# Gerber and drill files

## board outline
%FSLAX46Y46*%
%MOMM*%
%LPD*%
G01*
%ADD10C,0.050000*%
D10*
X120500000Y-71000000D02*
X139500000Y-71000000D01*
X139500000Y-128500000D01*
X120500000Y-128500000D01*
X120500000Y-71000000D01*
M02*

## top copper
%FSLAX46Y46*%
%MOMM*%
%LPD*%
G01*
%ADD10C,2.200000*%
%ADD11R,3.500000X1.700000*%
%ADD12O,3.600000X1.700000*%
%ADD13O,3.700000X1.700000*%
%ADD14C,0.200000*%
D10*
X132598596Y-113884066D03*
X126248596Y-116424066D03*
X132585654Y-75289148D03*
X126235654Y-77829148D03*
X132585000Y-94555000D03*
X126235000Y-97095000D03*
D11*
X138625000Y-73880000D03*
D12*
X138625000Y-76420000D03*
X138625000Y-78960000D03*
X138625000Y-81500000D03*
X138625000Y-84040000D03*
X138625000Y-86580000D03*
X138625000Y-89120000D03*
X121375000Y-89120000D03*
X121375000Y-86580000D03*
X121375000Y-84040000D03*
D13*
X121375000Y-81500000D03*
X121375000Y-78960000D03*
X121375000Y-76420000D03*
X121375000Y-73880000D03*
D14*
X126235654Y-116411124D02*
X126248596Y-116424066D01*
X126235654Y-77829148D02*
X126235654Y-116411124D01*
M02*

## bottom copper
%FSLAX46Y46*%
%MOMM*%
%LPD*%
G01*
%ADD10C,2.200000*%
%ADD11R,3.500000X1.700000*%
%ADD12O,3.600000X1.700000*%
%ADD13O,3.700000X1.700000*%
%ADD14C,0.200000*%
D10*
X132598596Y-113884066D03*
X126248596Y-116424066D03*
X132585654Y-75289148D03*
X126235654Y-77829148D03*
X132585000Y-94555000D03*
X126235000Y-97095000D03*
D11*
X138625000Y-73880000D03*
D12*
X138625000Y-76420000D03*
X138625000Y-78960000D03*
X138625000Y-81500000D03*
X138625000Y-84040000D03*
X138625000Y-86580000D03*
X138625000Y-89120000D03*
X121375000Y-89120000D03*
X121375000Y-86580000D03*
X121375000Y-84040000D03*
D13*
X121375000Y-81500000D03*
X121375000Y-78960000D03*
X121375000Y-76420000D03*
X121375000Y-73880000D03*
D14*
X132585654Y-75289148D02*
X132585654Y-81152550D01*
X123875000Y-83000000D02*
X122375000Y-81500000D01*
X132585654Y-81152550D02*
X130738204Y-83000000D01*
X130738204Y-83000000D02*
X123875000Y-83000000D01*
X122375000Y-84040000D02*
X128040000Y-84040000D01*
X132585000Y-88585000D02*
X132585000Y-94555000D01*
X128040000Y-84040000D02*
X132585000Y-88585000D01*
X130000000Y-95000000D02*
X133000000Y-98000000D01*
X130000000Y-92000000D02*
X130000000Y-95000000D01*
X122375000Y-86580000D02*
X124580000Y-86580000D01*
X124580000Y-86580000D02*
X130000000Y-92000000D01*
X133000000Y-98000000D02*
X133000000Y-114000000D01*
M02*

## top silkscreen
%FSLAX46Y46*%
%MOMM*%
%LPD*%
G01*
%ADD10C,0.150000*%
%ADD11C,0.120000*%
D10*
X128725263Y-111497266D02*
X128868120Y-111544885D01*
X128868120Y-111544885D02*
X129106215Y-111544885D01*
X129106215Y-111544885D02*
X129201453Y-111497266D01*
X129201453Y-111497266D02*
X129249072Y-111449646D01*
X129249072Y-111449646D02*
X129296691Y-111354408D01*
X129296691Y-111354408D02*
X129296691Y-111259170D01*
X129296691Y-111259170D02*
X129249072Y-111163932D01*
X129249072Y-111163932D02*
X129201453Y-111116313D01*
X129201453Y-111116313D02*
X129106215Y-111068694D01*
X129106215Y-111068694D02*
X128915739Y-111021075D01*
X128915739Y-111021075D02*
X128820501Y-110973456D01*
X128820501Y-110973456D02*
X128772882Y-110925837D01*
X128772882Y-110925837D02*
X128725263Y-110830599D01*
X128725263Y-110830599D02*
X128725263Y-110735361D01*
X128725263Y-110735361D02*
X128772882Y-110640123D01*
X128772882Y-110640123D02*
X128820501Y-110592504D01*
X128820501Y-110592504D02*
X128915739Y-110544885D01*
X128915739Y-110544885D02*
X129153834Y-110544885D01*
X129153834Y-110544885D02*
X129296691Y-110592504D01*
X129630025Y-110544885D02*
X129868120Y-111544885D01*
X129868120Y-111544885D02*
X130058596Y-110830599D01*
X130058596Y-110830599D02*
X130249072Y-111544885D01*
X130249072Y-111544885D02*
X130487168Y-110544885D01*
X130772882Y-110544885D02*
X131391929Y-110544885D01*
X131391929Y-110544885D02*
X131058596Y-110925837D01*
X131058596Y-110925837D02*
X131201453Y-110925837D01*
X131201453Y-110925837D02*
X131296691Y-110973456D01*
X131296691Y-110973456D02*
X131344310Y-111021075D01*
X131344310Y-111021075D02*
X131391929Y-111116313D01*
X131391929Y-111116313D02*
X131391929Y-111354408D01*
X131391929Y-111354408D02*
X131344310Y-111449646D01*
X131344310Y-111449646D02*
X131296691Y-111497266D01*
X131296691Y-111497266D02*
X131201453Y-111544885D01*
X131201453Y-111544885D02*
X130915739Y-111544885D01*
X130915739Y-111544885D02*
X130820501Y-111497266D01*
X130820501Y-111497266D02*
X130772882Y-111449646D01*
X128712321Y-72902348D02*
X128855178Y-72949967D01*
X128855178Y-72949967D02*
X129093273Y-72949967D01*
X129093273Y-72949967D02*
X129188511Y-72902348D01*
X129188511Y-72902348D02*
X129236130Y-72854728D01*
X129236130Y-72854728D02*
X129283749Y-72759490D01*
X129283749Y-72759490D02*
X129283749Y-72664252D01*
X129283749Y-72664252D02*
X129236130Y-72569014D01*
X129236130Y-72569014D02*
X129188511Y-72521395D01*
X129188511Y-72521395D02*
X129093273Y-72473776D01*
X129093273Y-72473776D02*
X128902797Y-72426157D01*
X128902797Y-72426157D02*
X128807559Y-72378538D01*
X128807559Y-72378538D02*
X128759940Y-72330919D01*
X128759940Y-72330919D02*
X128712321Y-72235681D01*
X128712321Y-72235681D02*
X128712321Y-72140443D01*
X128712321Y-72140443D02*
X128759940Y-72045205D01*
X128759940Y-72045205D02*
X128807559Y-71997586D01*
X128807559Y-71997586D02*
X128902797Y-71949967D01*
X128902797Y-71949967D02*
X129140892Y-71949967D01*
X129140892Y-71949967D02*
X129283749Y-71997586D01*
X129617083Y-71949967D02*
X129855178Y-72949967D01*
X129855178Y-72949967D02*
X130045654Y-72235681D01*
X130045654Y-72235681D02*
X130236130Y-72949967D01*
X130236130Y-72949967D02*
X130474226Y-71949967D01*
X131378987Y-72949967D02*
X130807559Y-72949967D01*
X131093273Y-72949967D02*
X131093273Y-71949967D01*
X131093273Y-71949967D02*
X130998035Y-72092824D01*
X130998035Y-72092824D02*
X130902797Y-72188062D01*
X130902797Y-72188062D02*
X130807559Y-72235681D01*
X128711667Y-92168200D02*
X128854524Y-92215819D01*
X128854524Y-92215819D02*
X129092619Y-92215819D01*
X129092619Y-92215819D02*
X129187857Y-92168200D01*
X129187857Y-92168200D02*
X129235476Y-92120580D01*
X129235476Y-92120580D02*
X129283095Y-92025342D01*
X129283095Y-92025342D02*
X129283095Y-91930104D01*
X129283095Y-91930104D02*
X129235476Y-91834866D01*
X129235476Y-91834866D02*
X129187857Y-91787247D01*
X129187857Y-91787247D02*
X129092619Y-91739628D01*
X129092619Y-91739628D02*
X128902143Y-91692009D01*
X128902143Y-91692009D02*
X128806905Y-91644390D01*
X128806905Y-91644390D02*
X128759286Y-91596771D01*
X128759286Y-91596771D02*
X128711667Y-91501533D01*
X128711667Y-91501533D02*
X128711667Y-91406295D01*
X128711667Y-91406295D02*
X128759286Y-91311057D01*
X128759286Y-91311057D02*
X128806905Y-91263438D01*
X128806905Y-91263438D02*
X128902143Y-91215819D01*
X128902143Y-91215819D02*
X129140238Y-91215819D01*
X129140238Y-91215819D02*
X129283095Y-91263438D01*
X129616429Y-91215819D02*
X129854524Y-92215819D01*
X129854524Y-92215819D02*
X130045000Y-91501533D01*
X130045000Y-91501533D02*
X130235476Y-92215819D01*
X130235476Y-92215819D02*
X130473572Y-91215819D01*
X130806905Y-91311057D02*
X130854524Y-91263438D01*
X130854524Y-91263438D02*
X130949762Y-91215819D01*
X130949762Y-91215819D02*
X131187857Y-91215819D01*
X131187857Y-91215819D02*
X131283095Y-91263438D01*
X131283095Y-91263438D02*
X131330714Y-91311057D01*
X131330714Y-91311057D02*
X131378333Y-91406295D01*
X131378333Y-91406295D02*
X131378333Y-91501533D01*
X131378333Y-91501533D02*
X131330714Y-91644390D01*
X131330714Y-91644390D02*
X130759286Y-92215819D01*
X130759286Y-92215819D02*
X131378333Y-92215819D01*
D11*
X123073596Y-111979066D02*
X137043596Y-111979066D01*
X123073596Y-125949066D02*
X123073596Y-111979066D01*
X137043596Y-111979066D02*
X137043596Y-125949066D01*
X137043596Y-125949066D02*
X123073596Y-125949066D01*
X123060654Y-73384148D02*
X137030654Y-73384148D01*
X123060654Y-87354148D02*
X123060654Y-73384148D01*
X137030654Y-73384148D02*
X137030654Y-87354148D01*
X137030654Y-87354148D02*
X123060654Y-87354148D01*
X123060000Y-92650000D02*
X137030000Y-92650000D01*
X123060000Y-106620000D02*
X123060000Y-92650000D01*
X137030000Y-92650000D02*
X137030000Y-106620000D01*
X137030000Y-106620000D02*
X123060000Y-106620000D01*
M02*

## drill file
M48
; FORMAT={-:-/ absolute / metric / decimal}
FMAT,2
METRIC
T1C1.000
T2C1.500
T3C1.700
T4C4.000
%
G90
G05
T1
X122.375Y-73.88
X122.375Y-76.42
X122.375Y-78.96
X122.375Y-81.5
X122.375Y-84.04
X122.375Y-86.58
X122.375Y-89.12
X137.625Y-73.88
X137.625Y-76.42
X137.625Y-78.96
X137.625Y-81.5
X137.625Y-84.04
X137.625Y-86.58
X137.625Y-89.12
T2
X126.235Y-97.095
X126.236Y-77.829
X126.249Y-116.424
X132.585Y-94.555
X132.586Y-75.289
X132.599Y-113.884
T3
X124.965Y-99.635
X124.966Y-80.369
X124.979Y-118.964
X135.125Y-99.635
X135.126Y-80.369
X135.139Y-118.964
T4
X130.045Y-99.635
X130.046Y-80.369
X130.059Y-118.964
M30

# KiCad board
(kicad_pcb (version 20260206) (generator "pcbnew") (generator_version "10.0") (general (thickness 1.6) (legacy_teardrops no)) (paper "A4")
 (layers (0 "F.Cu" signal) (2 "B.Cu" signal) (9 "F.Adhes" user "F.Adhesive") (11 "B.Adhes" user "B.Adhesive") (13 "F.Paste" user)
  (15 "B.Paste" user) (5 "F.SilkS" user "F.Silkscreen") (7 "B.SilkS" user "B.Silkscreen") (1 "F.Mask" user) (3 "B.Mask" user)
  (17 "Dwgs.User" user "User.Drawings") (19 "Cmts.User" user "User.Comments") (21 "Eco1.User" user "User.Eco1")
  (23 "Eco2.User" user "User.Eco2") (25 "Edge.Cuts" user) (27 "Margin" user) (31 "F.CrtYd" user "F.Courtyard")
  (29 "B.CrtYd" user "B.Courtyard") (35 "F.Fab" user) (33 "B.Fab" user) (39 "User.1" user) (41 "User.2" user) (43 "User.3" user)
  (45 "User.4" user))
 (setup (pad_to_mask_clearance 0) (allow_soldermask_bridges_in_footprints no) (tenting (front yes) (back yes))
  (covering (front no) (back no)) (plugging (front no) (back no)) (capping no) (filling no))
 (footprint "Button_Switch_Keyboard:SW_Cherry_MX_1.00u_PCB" (layer "F.Cu") (at 132.598596 113.884066)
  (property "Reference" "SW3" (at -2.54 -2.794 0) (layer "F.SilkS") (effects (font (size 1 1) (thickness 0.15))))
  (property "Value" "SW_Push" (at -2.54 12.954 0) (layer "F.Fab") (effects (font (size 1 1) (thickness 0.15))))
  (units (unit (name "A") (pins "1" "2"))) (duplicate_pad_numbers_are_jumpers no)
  (fp_line (start -9.525 -1.905) (end 4.445 -1.905) (stroke (width 0.12) (type solid)) (layer "F.SilkS"))
  (fp_line (start -9.525 12.065) (end -9.525 -1.905) (stroke (width 0.12) (type solid)) (layer "F.SilkS"))
  (fp_line (start 4.445 -1.905) (end 4.445 12.065) (stroke (width 0.12) (type solid)) (layer "F.SilkS"))
  (fp_line (start 4.445 12.065) (end -9.525 12.065) (stroke (width 0.12) (type solid)) (layer "F.SilkS"))
  (pad "" np_thru_hole circle (at -7.62 5.08) (size 1.7 1.7) (drill 1.7) (layers "*.Cu" "*.Mask"))
  (pad "" np_thru_hole circle (at -2.54 5.08) (size 4 4) (drill 4) (layers "*.Cu" "*.Mask"))
  (pad "" np_thru_hole circle (at 2.54 5.08) (size 1.7 1.7) (drill 1.7) (layers "*.Cu" "*.Mask"))
  (pad "1" thru_hole circle (at 0 0) (size 2.2 2.2) (drill 1.5) (layers "*.Cu" "*.Mask") (remove_unused_layers no)
   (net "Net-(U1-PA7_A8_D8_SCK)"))
  (pad "2" thru_hole circle (at -6.35 2.54) (size 2.2 2.2) (drill 1.5) (layers "*.Cu" "*.Mask") (remove_unused_layers no) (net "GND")))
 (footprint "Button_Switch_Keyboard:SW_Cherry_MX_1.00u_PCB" (layer "F.Cu") (at 132.585654 75.289148)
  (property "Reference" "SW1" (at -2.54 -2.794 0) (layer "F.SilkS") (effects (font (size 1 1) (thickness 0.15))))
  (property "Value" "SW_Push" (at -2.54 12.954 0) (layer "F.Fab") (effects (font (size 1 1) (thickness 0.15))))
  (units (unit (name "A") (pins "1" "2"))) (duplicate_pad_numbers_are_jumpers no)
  (fp_line (start -9.525 -1.905) (end 4.445 -1.905) (stroke (width 0.12) (type solid)) (layer "F.SilkS"))
  (fp_line (start -9.525 12.065) (end -9.525 -1.905) (stroke (width 0.12) (type solid)) (layer "F.SilkS"))
  (fp_line (start 4.445 -1.905) (end 4.445 12.065) (stroke (width 0.12) (type solid)) (layer "F.SilkS"))
  (fp_line (start 4.445 12.065) (end -9.525 12.065) (stroke (width 0.12) (type solid)) (layer "F.SilkS"))
  (pad "" np_thru_hole circle (at -7.62 5.08) (size 1.7 1.7) (drill 1.7) (layers "*.Cu" "*.Mask"))
  (pad "" np_thru_hole circle (at -2.54 5.08) (size 4 4) (drill 4) (layers "*.Cu" "*.Mask"))
  (pad "" np_thru_hole circle (at 2.54 5.08) (size 1.7 1.7) (drill 1.7) (layers "*.Cu" "*.Mask"))
  (pad "1" thru_hole circle (at 0 0) (size 2.2 2.2) (drill 1.5) (layers "*.Cu" "*.Mask") (remove_unused_layers no)
   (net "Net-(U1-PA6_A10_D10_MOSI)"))
  (pad "2" thru_hole circle (at -6.35 2.54) (size 2.2 2.2) (drill 1.5) (layers "*.Cu" "*.Mask") (remove_unused_layers no) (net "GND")))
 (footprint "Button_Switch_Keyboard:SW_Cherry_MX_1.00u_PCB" (layer "F.Cu") (at 132.585 94.555)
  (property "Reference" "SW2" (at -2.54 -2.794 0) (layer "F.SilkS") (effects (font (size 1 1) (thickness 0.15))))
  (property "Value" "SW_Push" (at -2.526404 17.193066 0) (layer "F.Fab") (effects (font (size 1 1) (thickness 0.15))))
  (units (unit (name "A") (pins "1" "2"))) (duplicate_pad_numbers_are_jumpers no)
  (fp_line (start -9.525 -1.905) (end 4.445 -1.905) (stroke (width 0.12) (type solid)) (layer "F.SilkS"))
  (fp_line (start -9.525 12.065) (end -9.525 -1.905) (stroke (width 0.12) (type solid)) (layer "F.SilkS"))
  (fp_line (start 4.445 -1.905) (end 4.445 12.065) (stroke (width 0.12) (type solid)) (layer "F.SilkS"))
  (fp_line (start 4.445 12.065) (end -9.525 12.065) (stroke (width 0.12) (type solid)) (layer "F.SilkS"))
  (pad "" np_thru_hole circle (at -7.62 5.08) (size 1.7 1.7) (drill 1.7) (layers "*.Cu" "*.Mask"))
  (pad "" np_thru_hole circle (at -2.54 5.08) (size 4 4) (drill 4) (layers "*.Cu" "*.Mask"))
  (pad "" np_thru_hole circle (at 2.54 5.08) (size 1.7 1.7) (drill 1.7) (layers "*.Cu" "*.Mask"))
  (pad "1" thru_hole circle (at 0 0) (size 2.2 2.2) (drill 1.5) (layers "*.Cu" "*.Mask") (remove_unused_layers no)
   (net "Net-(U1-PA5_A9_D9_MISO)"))
  (pad "2" thru_hole circle (at -6.35 2.54) (size 2.2 2.2) (drill 1.5) (layers "*.Cu" "*.Mask") (remove_unused_layers no) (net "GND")))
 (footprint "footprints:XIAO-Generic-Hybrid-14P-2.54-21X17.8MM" (layer "B.Cu") (at 130 81.5 180)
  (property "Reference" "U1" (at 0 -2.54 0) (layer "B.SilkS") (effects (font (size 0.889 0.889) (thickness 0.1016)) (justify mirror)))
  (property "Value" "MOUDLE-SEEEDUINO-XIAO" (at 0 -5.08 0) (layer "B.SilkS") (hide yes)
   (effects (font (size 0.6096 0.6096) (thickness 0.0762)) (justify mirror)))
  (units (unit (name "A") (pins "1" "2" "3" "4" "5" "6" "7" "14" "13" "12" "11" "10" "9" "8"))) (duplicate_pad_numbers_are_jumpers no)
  (pad "1" thru_hole rect (at -7.625 7.62 180) (size 3.5 1.7) (drill 1 (offset -1 0)) (layers "*.Cu" "*.Mask") (remove_unused_layers no)
   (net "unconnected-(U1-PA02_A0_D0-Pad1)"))
  (pad "2" thru_hole oval (at -7.625 5.08 180) (size 3.6 1.7) (drill 1 (offset -1 0)) (layers "*.Cu" "*.Mask") (remove_unused_layers no)
   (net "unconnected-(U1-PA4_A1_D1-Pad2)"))
  (pad "3" thru_hole oval (at -7.625 2.54 180) (size 3.6 1.7) (drill 1 (offset -1 0)) (layers "*.Cu" "*.Mask") (remove_unused_layers no)
   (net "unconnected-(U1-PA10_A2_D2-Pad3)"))
  (pad "4" thru_hole oval (at -7.625 0 180) (size 3.6 1.7) (drill 1 (offset -1 0)) (layers "*.Cu" "*.Mask") (remove_unused_layers no)
   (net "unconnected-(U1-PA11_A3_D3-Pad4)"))
  (pad "5" thru_hole oval (at -7.625 -2.54 180) (size 3.6 1.7) (drill 1 (offset -1 0)) (layers "*.Cu" "*.Mask") (remove_unused_layers no)
   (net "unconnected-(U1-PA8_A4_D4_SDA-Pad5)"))
  (pad "6" thru_hole oval (at -7.625 -5.08) (size 3.6 1.7) (drill 1 (offset 1 0)) (layers "*.Cu" "*.Mask") (remove_unused_layers no)
   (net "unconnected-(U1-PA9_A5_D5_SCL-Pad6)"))
  (pad "7" thru_hole oval (at -7.625 -7.62 180) (size 3.6 1.7) (drill 1 (offset -1 0)) (layers "*.Cu" "*.Mask") (remove_unused_layers no)
   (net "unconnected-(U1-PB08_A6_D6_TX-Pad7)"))
  (pad "8" thru_hole oval (at 7.625 -7.62 180) (size 3.6 1.7) (drill 1 (offset 1 0)) (layers "*.Cu" "*.Mask") (remove_unused_layers no)
   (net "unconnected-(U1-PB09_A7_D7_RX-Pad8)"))
  (pad "9" thru_hole oval (at 7.625 -5.08 180) (size 3.6 1.7) (drill 1 (offset 1 0)) (layers "*.Cu" "*.Mask") (remove_unused_layers no)
   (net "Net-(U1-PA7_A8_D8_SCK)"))
  (pad "10" thru_hole oval (at 7.625 -2.54 180) (size 3.6 1.7) (drill 1 (offset 1 0)) (layers "*.Cu" "*.Mask") (remove_unused_layers no)
   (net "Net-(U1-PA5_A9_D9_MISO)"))
  (pad "11" thru_hole oval (at 7.625 0 180) (size 3.7 1.7) (drill 1 (offset 1 0)) (layers "*.Cu" "*.Mask") (remove_unused_layers no)
   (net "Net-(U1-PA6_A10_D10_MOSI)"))
  (pad "12" thru_hole oval (at 7.625 2.54 180) (size 3.7 1.7) (drill 1 (offset 1 0)) (layers "*.Cu" "*.Mask") (remove_unused_layers no)
   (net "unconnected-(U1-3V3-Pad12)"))
  (pad "13" thru_hole oval (at 7.625 5.08 180) (size 3.7 1.7) (drill 1 (offset 1 0)) (layers "*.Cu" "*.Mask") (remove_unused_layers no)
   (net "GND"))
  (pad "14" thru_hole oval (at 7.625 7.62 180) (size 3.7 1.7) (drill 1 (offset 1 0)) (layers "*.Cu" "*.Mask") (remove_unused_layers no)
   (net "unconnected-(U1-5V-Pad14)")))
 (gr_rect (start 120.5 71) (end 139.5 128.5) (stroke (width 0.05) (type default)) (fill no) (layer "Edge.Cuts"))
 (segment (start 132.585654 75.289148) (end 132.585654 81.15255) (width 0.2) (layer "B.Cu") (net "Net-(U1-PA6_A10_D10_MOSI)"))
 (segment (start 123.875 83) (end 122.375 81.5) (width 0.2) (layer "B.Cu") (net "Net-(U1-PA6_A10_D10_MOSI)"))
 (segment (start 132.585654 81.15255) (end 130.738204 83) (width 0.2) (layer "B.Cu") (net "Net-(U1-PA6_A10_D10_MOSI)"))
 (segment (start 130.738204 83) (end 123.875 83) (width 0.2) (layer "B.Cu") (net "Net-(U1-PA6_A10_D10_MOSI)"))
 (segment (start 126.235654 116.411124) (end 126.248596 116.424066) (width 0.2) (layer "F.Cu") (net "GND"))
 (segment (start 126.235654 77.829148) (end 126.235654 116.411124) (width 0.2) (layer "F.Cu") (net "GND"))
 (segment (start 122.375 84.04) (end 128.04 84.04) (width 0.2) (layer "B.Cu") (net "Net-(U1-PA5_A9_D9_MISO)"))
 (segment (start 132.585 88.585) (end 132.585 94.555) (width 0.2) (layer "B.Cu") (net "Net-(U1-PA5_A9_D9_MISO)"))
 (segment (start 128.04 84.04) (end 132.585 88.585) (width 0.2) (layer "B.Cu") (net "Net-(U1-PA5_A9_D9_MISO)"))
 (segment (start 130 95) (end 133 98) (width 0.2) (layer "B.Cu") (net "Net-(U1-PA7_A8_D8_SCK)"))
 (segment (start 130 92) (end 130 95) (width 0.2) (layer "B.Cu") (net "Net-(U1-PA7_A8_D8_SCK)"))
 (segment (start 122.375 86.58) (end 124.58 86.58) (width 0.2) (layer "B.Cu") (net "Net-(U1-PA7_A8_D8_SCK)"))
 (segment (start 124.58 86.58) (end 130 92) (width 0.2) (layer "B.Cu") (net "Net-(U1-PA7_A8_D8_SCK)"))
 (segment (start 133 98) (end 133 114) (width 0.2) (layer "B.Cu") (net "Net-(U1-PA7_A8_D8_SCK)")))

